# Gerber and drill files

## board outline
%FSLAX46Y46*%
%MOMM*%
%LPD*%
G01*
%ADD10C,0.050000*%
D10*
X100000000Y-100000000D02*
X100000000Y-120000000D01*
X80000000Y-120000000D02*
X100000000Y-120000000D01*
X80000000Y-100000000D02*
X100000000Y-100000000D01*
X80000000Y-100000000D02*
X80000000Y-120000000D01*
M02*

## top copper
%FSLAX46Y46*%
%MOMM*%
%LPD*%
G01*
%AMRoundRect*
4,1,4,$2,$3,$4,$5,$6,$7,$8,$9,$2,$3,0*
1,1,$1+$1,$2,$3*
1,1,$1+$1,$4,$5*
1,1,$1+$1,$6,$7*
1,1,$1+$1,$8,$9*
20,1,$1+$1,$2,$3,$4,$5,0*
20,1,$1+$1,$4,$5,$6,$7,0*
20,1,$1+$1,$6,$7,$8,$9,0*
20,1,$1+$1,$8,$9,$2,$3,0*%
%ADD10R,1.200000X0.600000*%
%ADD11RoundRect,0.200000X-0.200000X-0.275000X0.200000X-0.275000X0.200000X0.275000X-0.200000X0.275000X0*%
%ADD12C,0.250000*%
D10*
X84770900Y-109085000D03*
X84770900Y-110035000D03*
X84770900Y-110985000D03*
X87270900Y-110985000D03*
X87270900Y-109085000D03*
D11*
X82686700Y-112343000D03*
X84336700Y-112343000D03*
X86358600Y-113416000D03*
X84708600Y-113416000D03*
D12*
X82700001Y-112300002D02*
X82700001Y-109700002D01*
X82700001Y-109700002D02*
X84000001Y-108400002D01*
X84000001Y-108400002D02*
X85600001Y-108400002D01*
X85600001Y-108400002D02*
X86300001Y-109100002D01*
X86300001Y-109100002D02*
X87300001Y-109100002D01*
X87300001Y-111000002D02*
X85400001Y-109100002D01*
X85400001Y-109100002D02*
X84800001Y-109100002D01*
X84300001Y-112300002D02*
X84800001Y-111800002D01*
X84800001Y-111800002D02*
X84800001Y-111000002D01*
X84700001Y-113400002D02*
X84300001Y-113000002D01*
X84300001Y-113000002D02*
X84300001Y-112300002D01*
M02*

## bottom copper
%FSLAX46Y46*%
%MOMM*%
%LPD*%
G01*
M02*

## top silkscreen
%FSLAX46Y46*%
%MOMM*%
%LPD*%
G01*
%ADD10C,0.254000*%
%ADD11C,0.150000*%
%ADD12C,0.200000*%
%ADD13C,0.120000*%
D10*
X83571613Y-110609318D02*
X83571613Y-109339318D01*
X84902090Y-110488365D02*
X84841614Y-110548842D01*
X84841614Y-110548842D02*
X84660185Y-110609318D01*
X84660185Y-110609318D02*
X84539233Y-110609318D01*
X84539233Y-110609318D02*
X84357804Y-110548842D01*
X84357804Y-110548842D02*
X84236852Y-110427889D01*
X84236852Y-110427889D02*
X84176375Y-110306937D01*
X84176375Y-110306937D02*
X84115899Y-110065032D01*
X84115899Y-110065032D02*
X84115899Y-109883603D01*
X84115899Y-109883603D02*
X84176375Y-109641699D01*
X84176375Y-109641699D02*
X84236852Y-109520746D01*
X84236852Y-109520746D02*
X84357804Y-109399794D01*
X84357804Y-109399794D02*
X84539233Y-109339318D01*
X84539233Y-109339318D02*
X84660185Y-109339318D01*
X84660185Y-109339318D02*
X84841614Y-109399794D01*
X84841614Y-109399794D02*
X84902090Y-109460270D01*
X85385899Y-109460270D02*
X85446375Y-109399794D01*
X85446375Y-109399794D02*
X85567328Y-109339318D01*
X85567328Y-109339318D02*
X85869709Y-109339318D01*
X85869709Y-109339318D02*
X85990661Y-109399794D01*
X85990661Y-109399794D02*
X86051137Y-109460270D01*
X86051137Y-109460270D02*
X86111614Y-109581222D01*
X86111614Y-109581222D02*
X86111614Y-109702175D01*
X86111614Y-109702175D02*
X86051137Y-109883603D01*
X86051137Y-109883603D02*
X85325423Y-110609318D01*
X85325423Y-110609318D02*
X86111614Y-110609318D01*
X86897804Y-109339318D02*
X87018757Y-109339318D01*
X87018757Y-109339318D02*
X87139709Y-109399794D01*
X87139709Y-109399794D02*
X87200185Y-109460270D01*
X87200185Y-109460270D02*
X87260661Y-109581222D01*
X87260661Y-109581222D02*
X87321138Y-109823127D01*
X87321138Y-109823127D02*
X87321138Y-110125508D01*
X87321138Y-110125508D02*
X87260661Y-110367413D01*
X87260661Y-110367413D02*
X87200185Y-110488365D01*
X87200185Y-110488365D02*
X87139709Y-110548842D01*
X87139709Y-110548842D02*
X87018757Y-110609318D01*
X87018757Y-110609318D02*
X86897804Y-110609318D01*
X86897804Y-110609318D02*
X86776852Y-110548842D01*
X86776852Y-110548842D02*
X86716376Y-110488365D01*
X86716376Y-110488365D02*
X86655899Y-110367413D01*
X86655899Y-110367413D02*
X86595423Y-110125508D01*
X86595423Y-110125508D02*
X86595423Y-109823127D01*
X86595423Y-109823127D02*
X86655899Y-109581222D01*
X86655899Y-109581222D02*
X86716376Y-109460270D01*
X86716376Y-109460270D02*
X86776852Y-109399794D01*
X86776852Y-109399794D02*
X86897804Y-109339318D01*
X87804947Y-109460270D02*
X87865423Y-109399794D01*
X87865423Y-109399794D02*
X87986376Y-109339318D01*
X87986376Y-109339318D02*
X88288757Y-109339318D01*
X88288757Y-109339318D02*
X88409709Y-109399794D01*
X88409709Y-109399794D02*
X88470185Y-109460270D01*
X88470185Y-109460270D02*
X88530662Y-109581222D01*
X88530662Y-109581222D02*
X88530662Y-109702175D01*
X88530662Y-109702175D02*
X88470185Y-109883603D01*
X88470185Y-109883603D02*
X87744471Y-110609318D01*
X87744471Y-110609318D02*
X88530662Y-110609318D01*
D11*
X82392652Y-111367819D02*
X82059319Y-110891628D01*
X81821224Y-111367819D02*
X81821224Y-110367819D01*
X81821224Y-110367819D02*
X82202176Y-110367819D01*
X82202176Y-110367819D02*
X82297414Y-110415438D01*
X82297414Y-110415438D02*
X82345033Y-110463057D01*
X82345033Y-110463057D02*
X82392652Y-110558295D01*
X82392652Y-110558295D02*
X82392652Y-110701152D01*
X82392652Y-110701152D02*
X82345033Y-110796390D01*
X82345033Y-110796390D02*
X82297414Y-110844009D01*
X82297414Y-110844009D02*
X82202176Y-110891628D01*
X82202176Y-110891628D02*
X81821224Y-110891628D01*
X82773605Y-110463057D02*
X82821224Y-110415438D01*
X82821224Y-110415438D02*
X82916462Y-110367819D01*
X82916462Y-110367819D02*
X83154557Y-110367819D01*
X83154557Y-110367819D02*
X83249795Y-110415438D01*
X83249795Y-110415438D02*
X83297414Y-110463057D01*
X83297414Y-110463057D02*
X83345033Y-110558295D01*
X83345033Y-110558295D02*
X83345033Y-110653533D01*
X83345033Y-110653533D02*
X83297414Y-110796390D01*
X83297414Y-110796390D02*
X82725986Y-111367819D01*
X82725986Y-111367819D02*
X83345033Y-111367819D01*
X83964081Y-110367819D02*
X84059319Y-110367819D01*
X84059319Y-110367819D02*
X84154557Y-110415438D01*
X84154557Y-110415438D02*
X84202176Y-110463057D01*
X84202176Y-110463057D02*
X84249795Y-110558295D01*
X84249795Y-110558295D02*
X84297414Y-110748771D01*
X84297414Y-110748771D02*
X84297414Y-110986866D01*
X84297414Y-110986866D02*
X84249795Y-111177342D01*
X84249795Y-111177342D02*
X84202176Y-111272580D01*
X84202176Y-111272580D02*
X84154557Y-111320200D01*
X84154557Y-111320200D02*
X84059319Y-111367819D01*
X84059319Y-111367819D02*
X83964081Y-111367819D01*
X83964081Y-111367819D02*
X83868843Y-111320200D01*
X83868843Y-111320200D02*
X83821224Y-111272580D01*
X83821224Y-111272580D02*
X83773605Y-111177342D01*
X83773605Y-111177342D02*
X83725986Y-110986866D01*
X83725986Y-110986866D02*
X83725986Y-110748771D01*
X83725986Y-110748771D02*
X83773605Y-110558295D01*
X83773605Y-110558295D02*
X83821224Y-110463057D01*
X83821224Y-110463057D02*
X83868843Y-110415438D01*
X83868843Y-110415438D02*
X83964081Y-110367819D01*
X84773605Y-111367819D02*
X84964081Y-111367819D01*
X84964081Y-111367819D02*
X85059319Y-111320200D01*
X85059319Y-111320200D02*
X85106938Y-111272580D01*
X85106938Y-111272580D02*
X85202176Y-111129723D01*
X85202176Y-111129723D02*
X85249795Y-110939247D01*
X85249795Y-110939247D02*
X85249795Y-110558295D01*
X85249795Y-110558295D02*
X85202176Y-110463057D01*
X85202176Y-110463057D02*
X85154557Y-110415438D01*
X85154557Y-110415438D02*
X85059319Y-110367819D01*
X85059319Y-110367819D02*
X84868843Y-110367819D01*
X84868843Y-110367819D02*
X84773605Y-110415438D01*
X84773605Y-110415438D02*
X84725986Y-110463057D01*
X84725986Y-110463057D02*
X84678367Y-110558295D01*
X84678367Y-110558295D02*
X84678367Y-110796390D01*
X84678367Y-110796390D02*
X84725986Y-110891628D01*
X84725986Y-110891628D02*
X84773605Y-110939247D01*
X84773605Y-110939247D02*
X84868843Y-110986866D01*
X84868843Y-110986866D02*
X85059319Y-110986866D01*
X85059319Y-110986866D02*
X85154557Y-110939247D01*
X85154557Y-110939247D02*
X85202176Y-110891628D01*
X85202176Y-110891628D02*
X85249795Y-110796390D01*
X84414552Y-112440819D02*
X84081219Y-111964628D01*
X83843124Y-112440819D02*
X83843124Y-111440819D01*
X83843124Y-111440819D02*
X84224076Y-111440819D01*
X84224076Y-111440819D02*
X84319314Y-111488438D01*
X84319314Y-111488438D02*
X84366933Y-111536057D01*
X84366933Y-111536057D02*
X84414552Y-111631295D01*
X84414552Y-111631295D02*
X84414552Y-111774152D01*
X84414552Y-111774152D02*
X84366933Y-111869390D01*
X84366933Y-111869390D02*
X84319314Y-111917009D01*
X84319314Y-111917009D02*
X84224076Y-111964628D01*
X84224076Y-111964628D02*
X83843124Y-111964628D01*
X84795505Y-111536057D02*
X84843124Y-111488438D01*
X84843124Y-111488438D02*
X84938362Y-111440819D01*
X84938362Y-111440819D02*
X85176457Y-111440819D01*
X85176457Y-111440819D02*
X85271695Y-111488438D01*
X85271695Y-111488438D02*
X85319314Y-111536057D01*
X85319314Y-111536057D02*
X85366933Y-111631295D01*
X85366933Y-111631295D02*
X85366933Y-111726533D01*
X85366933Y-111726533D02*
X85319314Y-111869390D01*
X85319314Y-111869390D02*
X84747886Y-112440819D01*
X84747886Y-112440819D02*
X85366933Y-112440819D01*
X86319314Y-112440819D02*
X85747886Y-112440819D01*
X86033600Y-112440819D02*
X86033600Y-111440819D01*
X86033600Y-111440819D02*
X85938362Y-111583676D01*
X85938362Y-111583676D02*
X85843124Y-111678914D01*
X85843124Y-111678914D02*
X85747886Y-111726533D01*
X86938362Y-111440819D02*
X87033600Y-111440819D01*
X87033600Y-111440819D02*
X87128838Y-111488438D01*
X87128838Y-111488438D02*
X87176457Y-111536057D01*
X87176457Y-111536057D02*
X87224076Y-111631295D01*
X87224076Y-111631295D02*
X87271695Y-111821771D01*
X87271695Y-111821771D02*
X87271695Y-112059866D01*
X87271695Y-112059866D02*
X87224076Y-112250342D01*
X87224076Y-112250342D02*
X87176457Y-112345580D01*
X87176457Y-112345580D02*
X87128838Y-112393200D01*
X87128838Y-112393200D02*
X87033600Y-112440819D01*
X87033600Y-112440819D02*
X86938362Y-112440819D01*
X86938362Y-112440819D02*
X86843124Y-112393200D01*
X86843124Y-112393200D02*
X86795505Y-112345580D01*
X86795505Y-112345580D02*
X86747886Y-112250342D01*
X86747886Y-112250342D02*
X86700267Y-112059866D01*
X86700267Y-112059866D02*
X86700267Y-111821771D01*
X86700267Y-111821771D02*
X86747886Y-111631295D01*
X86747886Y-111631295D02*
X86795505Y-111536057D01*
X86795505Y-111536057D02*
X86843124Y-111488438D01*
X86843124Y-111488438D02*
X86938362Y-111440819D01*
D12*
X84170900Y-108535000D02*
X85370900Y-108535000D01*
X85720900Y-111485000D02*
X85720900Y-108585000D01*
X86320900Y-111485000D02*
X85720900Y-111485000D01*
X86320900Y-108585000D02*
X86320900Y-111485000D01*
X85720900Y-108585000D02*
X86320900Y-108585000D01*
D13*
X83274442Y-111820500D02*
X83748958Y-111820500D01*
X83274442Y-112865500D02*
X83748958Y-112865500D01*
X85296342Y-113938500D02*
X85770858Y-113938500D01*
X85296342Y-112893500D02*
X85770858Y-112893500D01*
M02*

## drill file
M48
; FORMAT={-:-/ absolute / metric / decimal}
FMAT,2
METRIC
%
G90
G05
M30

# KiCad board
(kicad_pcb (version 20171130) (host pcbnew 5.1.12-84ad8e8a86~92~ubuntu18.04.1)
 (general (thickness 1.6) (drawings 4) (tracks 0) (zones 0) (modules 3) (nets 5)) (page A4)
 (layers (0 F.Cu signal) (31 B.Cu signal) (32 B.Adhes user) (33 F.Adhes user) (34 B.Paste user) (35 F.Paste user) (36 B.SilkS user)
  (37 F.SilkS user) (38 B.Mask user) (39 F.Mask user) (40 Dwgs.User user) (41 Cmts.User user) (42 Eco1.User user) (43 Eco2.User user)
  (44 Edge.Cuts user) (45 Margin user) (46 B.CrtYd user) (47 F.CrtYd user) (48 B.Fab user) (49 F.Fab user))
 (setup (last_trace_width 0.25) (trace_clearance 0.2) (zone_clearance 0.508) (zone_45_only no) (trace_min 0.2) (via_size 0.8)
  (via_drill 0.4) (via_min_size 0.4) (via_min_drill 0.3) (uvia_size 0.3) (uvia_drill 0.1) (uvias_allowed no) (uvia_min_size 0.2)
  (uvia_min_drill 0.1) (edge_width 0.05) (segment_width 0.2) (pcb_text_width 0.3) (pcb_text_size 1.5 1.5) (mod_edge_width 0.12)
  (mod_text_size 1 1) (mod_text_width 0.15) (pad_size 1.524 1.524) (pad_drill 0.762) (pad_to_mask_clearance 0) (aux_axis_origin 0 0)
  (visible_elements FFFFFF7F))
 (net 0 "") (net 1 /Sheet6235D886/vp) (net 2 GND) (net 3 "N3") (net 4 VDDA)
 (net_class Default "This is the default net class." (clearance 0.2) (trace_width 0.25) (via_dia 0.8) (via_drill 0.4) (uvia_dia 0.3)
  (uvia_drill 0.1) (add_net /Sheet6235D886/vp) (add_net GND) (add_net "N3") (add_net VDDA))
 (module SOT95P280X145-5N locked (layer F.Cu) (at 86.020900 110.035000)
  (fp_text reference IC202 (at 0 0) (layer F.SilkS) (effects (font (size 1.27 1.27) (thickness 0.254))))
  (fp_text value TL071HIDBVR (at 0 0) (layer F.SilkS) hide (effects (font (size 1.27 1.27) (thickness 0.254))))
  (fp_line (start -1.85 -1.5) (end -0.65 -1.5) (layer F.SilkS) (width 0.2))
  (fp_line (start -0.3 1.45) (end -0.3 -1.45) (layer F.SilkS) (width 0.2))
  (fp_line (start 0.3 1.45) (end -0.3 1.45) (layer F.SilkS) (width 0.2))
  (fp_line (start 0.3 -1.45) (end 0.3 1.45) (layer F.SilkS) (width 0.2))
  (fp_line (start -0.3 -1.45) (end 0.3 -1.45) (layer F.SilkS) (width 0.2))
  (pad 1 smd rect (at -1.25 -0.95 90.000000) (size 0.6 1.2) (layers F.Cu F.Mask F.Paste) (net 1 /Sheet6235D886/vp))
  (pad 2 smd rect (at -1.25 0 90.000000) (size 0.6 1.2) (layers F.Cu F.Mask F.Paste) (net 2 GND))
  (pad 3 smd rect (at -1.25 0.95 90.000000) (size 0.6 1.2) (layers F.Cu F.Mask F.Paste) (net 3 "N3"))
  (pad 4 smd rect (at 1.25 0.95 90.000000) (size 0.6 1.2) (layers F.Cu F.Mask F.Paste) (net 1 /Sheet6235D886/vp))
  (pad 5 smd rect (at 1.25 -0.95 90.000000) (size 0.6 1.2) (layers F.Cu F.Mask F.Paste) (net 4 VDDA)))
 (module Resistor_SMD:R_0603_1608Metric (layer F.Cu) (at 83.511700 112.343000)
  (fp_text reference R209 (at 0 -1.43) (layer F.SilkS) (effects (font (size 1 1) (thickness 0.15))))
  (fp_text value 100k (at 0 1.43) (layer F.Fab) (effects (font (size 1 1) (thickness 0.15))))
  (fp_line (start -0.237258 -0.5225) (end 0.237258 -0.5225) (layer F.SilkS) (width 0.12))
  (fp_line (start -0.237258 0.5225) (end 0.237258 0.5225) (layer F.SilkS) (width 0.12))
  (pad 1 smd roundrect (at -0.825 0) (size 0.8 0.95) (layers F.Cu F.Mask F.Paste) (roundrect_rratio 0.25) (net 4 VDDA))
  (pad 2 smd roundrect (at 0.825 0) (size 0.8 0.95) (layers F.Cu F.Mask F.Paste) (roundrect_rratio 0.25) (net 3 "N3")))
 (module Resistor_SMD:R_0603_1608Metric (layer F.Cu) (at 85.533600 113.416000)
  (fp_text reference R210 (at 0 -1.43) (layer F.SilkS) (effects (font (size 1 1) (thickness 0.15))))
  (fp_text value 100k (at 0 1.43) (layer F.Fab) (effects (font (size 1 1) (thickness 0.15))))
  (fp_line (start -0.237258 0.5225) (end 0.237258 0.5225) (layer F.SilkS) (width 0.12))
  (fp_line (start -0.237258 -0.5225) (end 0.237258 -0.5225) (layer F.SilkS) (width 0.12))
  (pad 2 smd roundrect (at 0.825 0) (size 0.8 0.95) (layers F.Cu F.Mask F.Paste) (roundrect_rratio 0.25) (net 2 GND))
  (pad 1 smd roundrect (at -0.825 0) (size 0.8 0.95) (layers F.Cu F.Mask F.Paste) (roundrect_rratio 0.25) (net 3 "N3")))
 (gr_line (start 100 100) (end 100 120) (layer Edge.Cuts) (width 0.05))
 (gr_line (start 80 120) (end 100 120) (layer Edge.Cuts) (width 0.05))
 (gr_line (start 80 100) (end 100 100) (layer Edge.Cuts) (width 0.05))
 (gr_line (start 80 100) (end 80 120) (layer Edge.Cuts) (width 0.05))
 (segment (start 82.700001 112.300002) (end 82.700001 109.700002) (width 0.250000) (layer F.Cu) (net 4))
 (segment (start 82.700001 109.700002) (end 84.000001 108.400002) (width 0.250000) (layer F.Cu) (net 4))
 (segment (start 84.000001 108.400002) (end 85.600001 108.400002) (width 0.250000) (layer F.Cu) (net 4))
 (segment (start 85.600001 108.400002) (end 86.300001 109.100002) (width 0.250000) (layer F.Cu) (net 4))
 (segment (start 86.300001 109.100002) (end 87.300001 109.100002) (width 0.250000) (layer F.Cu) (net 4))
 (segment (start 87.300001 111.000002) (end 85.400001 109.100002) (width 0.250000) (layer F.Cu) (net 1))
 (segment (start 85.400001 109.100002) (end 84.800001 109.100002) (width 0.250000) (layer F.Cu) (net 1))
 (segment (start 84.300001 112.300002) (end 84.800001 111.800002) (width 0.250000) (layer F.Cu) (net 3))
 (segment (start 84.800001 111.800002) (end 84.800001 111.000002) (width 0.250000) (layer F.Cu) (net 3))
 (segment (start 84.700001 113.400002) (end 84.300001 113.000002) (width 0.250000) (layer F.Cu) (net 3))
 (segment (start 84.300001 113.000002) (end 84.300001 112.300002) (width 0.250000) (layer F.Cu) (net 3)))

